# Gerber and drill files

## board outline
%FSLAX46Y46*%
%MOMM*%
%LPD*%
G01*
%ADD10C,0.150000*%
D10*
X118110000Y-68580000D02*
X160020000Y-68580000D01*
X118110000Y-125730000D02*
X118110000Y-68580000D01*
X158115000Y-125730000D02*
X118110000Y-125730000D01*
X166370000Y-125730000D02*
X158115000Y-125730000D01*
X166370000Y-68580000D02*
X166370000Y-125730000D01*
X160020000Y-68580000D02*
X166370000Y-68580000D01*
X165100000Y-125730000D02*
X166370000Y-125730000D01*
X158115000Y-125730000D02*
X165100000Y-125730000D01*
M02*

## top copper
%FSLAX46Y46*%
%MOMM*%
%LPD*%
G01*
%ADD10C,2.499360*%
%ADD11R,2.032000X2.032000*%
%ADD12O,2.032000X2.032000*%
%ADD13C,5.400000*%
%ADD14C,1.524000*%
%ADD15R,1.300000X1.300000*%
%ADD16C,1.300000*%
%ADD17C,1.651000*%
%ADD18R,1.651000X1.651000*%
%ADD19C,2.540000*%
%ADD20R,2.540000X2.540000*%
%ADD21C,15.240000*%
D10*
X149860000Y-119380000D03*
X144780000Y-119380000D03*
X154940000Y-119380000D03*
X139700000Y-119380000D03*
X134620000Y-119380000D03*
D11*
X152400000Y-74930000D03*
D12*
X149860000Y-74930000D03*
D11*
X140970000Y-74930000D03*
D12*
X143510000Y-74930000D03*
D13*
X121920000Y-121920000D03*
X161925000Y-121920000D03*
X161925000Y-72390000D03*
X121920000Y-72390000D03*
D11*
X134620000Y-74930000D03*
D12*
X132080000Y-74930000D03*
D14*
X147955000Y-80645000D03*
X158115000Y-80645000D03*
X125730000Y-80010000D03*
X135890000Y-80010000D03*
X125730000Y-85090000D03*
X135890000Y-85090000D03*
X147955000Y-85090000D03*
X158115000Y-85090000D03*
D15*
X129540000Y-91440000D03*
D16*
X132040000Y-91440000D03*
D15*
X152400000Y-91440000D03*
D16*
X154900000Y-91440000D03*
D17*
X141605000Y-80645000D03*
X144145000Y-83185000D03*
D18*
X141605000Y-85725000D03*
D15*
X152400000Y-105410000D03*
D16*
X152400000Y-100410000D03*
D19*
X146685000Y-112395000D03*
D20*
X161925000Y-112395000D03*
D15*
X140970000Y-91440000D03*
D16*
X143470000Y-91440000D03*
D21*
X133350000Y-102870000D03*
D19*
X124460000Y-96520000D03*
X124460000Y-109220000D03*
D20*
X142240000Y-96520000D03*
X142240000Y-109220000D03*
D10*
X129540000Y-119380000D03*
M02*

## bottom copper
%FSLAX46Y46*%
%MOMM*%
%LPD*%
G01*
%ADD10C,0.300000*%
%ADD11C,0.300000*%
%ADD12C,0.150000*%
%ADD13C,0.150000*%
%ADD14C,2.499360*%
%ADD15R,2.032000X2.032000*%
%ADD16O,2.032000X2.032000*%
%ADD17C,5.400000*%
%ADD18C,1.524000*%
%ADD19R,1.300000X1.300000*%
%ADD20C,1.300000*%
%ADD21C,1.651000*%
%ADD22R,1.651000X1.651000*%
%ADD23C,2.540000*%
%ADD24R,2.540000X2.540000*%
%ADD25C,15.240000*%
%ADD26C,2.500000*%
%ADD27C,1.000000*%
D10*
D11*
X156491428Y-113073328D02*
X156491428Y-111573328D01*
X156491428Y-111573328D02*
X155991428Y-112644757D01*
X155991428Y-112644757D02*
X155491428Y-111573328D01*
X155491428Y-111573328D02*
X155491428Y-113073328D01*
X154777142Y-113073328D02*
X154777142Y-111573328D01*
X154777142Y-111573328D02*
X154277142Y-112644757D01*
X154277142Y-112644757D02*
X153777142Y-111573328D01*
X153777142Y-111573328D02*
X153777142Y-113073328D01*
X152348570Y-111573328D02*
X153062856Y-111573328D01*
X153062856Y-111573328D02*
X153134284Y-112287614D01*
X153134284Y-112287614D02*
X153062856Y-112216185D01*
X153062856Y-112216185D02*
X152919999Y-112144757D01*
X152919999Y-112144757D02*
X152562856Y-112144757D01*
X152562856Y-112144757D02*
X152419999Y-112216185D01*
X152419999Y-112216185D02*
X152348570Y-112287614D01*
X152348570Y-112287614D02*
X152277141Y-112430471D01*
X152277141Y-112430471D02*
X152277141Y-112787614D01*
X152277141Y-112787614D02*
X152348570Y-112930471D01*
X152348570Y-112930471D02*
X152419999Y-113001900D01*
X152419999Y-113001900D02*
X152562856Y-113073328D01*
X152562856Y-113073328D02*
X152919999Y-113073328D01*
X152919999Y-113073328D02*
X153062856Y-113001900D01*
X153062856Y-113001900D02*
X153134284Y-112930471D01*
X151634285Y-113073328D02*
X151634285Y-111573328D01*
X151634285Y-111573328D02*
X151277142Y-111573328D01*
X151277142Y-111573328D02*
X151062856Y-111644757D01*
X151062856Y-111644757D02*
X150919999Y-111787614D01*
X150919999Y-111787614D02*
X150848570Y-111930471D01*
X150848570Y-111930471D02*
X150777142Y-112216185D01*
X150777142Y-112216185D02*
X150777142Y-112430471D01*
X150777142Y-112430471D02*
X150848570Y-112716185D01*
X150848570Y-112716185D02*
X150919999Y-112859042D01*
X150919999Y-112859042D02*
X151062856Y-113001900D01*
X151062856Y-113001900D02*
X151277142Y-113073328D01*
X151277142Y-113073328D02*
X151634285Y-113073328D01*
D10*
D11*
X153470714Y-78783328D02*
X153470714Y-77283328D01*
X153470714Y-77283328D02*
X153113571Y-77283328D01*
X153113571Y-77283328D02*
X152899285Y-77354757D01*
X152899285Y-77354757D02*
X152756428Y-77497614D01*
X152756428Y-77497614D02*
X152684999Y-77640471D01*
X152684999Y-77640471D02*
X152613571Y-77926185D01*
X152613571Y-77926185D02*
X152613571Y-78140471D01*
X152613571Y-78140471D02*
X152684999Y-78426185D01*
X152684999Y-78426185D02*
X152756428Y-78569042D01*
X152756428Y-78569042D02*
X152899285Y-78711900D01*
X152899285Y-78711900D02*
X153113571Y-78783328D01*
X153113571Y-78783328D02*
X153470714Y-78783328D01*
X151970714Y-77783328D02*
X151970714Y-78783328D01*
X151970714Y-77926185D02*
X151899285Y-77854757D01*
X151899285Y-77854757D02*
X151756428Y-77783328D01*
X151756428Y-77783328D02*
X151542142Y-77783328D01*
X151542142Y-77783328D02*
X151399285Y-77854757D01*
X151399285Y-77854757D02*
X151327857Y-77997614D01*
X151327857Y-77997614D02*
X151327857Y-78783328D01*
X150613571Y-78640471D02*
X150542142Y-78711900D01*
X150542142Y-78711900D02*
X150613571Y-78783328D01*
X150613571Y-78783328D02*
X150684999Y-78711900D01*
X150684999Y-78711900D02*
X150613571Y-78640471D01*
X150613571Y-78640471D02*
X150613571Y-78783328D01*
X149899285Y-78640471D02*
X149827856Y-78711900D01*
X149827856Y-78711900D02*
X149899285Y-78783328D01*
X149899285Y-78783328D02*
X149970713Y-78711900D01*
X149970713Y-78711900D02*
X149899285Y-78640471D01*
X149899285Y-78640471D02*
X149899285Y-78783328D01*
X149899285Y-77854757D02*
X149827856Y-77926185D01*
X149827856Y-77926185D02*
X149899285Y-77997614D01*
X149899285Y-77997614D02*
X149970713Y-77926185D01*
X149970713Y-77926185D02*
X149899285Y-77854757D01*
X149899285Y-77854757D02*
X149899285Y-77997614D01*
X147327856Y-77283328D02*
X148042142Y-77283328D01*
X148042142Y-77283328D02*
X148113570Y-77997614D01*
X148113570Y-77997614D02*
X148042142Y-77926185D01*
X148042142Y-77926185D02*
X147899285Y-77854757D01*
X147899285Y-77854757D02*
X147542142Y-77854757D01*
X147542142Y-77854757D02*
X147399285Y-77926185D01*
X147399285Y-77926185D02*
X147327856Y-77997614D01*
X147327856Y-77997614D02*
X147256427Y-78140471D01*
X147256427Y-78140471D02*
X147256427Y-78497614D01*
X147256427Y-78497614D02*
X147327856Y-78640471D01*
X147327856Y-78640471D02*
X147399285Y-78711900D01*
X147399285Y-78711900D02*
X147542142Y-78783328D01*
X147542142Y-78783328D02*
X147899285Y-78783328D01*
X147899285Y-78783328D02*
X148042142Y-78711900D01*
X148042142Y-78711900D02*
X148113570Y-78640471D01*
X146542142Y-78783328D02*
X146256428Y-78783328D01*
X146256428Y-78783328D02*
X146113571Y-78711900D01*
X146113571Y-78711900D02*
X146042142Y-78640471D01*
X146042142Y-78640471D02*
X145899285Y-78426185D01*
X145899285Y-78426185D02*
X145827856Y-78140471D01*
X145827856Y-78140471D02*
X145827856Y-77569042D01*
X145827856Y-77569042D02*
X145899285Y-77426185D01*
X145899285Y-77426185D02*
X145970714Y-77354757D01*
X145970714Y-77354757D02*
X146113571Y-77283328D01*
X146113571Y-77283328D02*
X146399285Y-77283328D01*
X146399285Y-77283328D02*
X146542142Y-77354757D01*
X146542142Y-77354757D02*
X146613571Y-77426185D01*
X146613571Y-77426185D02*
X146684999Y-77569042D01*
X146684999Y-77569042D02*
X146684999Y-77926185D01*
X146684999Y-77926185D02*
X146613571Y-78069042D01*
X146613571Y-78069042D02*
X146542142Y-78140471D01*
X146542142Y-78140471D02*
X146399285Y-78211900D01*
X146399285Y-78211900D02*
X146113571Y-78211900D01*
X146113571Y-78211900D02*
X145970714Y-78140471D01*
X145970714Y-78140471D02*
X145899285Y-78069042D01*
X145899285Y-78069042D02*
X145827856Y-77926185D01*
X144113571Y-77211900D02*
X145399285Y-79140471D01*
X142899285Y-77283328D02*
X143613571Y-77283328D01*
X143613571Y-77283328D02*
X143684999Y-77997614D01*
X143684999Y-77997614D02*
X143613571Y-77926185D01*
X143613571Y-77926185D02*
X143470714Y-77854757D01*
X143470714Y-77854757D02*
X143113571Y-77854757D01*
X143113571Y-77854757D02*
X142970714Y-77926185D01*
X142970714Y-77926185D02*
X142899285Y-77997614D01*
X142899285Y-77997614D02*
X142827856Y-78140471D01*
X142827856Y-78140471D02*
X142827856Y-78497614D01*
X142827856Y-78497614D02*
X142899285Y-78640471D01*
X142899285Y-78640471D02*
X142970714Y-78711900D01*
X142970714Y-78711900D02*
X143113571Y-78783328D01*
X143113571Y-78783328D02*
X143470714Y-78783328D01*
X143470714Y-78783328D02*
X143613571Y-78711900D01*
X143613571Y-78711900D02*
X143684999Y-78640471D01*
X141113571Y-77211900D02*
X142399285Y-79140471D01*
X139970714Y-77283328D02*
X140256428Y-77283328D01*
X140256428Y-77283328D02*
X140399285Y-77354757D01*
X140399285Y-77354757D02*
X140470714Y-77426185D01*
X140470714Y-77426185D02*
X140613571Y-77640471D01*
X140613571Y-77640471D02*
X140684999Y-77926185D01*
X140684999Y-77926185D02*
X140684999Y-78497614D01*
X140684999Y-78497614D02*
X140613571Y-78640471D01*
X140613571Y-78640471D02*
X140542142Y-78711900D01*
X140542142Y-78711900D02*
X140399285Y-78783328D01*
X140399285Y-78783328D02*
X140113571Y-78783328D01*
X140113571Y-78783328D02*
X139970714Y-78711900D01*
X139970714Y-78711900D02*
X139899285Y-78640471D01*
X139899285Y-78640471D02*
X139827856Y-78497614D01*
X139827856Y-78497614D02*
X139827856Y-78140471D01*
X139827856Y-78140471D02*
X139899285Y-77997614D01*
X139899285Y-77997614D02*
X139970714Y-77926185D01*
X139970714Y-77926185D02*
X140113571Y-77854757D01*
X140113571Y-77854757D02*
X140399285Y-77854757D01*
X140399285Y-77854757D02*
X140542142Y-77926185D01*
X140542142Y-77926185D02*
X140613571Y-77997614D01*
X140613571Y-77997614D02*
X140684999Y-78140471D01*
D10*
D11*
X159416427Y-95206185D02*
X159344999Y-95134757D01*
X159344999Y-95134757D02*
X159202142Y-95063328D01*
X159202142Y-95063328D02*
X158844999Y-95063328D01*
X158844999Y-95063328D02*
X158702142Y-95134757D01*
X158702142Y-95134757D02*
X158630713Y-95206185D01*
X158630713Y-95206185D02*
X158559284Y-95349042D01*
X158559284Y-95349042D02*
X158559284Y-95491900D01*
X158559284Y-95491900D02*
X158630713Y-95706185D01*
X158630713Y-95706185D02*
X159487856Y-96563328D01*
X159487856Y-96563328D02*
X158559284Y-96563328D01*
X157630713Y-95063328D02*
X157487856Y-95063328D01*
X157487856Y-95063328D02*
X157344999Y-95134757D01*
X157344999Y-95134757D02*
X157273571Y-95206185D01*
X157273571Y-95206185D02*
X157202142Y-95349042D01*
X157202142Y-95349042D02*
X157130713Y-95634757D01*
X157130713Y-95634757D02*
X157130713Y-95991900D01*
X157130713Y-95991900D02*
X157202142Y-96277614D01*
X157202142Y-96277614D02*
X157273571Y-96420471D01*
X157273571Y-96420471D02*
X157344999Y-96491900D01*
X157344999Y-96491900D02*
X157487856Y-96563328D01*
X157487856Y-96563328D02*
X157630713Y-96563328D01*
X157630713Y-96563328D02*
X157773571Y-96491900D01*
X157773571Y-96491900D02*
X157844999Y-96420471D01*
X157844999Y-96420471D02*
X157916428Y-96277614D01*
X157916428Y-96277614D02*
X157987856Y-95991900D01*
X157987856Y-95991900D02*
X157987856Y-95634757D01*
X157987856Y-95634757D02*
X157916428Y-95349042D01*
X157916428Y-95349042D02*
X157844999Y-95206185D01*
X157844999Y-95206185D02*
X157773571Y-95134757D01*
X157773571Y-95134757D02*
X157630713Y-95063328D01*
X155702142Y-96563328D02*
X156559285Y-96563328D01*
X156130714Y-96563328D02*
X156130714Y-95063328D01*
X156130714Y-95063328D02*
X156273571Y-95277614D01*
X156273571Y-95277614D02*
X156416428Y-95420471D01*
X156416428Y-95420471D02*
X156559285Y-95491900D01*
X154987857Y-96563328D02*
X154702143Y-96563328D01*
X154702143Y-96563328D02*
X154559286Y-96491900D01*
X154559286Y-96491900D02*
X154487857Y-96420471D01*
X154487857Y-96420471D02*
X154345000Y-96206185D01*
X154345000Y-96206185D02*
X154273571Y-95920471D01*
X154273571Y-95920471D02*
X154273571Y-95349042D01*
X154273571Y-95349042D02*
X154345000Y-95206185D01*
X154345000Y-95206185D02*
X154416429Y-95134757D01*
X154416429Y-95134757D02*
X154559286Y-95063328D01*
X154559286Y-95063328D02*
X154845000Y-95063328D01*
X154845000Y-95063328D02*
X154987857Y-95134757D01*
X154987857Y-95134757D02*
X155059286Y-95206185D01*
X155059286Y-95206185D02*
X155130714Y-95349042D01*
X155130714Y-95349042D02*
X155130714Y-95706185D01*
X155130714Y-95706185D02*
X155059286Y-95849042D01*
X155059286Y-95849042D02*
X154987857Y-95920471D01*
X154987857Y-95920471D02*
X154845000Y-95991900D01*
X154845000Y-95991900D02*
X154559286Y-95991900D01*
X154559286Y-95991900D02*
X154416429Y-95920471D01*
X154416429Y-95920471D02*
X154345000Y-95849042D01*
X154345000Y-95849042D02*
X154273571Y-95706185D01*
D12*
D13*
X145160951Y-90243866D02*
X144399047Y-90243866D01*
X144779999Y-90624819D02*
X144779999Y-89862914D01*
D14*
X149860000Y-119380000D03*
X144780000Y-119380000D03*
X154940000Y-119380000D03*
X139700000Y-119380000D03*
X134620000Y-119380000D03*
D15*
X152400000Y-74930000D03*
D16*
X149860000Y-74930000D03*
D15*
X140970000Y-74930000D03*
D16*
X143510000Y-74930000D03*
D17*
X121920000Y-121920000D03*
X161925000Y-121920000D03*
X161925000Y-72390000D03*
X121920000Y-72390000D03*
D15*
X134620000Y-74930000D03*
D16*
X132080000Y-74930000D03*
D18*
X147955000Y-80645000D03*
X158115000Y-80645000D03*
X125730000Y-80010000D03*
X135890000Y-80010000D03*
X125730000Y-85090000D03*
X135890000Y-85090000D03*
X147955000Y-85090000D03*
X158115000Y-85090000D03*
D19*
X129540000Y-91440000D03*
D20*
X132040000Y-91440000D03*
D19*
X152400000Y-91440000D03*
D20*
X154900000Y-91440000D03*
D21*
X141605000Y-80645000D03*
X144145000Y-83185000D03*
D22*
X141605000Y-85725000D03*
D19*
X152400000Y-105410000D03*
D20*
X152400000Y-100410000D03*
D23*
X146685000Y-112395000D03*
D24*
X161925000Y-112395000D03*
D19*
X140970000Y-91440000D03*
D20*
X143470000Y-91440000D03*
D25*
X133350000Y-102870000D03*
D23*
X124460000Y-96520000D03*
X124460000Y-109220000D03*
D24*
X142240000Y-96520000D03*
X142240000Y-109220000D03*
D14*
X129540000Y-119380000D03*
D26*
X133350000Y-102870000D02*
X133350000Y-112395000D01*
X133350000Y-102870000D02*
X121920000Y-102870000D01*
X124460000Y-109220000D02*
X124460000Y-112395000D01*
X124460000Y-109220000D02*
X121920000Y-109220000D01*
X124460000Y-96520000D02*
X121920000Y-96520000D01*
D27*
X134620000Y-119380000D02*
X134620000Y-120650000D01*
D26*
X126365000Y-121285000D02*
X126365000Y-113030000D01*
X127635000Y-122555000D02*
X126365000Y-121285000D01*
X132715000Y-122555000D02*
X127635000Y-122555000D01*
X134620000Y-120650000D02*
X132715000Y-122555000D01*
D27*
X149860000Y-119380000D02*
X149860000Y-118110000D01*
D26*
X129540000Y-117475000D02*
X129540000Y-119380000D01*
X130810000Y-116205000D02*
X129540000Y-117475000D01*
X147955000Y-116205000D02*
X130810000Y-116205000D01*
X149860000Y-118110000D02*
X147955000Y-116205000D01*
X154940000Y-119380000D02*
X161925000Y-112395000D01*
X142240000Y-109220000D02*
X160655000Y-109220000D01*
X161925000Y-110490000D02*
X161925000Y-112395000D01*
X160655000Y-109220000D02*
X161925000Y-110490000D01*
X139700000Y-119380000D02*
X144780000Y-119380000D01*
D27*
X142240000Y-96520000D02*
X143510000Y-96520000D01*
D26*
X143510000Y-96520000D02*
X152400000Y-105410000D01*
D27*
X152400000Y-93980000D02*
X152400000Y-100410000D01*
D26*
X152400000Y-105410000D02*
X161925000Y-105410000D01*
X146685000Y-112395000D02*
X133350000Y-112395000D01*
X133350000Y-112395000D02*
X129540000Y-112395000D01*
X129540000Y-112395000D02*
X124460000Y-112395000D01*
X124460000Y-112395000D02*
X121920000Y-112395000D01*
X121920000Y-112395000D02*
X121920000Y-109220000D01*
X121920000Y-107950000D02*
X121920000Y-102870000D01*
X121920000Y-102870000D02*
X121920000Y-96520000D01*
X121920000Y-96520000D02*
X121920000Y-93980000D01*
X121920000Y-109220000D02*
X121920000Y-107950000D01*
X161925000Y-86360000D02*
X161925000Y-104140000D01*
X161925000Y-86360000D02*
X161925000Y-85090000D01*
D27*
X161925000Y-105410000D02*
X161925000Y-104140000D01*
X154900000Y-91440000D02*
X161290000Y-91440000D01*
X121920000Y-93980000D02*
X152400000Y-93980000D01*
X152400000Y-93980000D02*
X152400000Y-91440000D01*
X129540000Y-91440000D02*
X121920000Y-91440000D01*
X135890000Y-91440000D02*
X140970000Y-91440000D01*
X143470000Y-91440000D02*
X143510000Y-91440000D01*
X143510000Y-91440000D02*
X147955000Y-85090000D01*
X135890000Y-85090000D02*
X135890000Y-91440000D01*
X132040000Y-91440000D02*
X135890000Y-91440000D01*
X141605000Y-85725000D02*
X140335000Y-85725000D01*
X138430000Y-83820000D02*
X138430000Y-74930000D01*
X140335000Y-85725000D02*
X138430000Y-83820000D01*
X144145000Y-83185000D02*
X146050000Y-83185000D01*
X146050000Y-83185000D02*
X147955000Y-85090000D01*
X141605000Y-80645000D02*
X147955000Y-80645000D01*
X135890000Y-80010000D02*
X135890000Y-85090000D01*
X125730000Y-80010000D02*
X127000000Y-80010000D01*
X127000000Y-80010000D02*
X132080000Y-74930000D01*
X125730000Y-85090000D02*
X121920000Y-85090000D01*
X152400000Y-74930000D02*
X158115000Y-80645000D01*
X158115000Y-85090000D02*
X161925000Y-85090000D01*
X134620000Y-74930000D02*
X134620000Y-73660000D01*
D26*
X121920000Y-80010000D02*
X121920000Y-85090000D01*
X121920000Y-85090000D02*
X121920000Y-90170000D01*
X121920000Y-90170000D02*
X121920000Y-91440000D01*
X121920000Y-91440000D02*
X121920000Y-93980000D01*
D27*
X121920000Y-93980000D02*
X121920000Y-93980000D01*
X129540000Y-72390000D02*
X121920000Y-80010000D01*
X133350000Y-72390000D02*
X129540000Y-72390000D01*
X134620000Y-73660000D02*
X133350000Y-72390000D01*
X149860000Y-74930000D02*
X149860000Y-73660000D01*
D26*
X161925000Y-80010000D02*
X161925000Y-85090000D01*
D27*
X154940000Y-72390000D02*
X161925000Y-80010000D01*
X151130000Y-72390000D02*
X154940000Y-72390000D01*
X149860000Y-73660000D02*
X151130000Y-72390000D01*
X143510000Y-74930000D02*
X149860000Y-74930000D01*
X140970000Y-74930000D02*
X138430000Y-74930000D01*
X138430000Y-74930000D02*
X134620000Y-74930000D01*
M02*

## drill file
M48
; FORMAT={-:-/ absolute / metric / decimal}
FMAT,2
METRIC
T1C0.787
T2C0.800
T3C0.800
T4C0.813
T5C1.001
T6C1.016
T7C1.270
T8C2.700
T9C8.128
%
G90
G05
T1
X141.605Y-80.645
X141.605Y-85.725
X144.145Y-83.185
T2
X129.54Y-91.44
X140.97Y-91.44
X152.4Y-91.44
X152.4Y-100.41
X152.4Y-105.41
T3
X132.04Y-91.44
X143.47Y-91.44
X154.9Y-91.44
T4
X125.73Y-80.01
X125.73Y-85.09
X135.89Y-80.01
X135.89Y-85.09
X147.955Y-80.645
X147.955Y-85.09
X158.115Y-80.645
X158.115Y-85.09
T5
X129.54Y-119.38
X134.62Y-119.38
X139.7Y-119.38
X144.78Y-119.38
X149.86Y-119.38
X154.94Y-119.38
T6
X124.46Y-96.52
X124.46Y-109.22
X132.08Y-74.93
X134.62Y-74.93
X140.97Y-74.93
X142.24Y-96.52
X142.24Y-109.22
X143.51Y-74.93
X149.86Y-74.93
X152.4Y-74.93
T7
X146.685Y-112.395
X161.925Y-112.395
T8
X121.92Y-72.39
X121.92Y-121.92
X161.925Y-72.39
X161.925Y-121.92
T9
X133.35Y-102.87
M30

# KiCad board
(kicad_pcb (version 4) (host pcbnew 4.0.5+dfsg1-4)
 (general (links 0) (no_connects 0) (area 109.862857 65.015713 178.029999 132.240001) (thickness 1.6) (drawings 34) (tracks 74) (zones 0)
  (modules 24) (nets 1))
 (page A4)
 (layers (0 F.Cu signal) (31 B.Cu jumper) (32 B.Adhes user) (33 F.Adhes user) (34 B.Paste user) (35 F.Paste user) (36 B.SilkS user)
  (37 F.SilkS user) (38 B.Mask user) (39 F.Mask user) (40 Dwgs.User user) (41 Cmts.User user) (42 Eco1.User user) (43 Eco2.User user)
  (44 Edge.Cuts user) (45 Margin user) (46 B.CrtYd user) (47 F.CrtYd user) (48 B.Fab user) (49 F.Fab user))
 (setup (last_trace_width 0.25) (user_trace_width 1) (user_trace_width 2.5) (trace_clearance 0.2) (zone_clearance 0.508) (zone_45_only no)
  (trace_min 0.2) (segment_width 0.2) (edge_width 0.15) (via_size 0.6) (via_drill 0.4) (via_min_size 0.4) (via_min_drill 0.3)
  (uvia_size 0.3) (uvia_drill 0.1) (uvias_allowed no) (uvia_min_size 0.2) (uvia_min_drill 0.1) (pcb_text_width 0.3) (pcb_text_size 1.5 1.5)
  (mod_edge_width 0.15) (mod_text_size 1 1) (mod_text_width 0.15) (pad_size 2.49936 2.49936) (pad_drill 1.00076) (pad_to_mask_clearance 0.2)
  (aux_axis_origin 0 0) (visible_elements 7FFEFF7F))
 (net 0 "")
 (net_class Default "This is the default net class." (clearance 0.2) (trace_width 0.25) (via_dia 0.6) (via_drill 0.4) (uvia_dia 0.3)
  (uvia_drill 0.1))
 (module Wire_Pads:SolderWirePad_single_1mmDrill (layer F.Cu) (at 149.86 119.38)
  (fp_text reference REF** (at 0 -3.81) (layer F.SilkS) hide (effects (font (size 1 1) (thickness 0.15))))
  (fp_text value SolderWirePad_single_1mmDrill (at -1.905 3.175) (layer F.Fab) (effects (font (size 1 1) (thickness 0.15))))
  (pad 2 thru_hole circle (at 0 0) (size 2.49936 2.49936) (drill 1.00076) (layers *.Cu *.Mask)))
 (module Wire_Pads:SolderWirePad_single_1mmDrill (layer F.Cu) (at 144.78 119.38)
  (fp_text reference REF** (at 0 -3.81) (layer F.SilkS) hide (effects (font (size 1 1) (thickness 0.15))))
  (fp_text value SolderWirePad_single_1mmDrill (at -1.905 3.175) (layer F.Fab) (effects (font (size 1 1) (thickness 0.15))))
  (pad 1 thru_hole circle (at 0 0) (size 2.49936 2.49936) (drill 1.00076) (layers *.Cu *.Mask)))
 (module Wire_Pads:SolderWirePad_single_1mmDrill (layer F.Cu) (at 154.94 119.38)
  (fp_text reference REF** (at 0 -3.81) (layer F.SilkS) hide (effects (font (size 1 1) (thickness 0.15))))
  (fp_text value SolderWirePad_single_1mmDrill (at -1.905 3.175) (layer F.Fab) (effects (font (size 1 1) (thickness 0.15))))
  (pad 3 thru_hole circle (at 0 0) (size 2.49936 2.49936) (drill 1.00076) (layers *.Cu *.Mask)))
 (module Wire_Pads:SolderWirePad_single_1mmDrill (layer F.Cu) (at 139.7 119.38)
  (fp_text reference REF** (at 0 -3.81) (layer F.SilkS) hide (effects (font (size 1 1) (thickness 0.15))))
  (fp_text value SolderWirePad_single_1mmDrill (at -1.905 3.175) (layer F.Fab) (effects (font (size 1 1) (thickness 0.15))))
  (pad 3 thru_hole circle (at 0 0) (size 2.49936 2.49936) (drill 1.00076) (layers *.Cu *.Mask)))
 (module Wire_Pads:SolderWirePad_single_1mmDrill (layer F.Cu) (at 134.62 119.38)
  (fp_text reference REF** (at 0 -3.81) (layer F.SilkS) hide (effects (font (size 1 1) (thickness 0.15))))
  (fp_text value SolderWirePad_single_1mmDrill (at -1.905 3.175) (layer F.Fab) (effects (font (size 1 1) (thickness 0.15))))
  (pad 2 thru_hole circle (at 0 0) (size 2.49936 2.49936) (drill 1.00076) (layers *.Cu *.Mask)))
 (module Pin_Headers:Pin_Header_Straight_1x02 (layer F.Cu) (at 152.4 74.93 270)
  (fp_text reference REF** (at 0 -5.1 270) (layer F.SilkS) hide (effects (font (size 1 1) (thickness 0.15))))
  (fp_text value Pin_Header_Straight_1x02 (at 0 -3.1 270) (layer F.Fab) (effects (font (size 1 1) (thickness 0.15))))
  (pad 1 thru_hole rect (at 0 0 270) (size 2.032 2.032) (drill 1.016) (layers *.Cu *.Mask))
  (pad 2 thru_hole oval (at 0 2.54 270) (size 2.032 2.032) (drill 1.016) (layers *.Cu *.Mask)))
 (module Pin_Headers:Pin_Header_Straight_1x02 (layer F.Cu) (at 140.97 74.93 90)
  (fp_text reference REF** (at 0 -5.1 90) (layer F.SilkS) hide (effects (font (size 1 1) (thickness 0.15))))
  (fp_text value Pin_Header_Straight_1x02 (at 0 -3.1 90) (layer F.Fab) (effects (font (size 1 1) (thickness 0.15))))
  (pad 1 thru_hole rect (at 0 0 90) (size 2.032 2.032) (drill 1.016) (layers *.Cu *.Mask))
  (pad 2 thru_hole oval (at 0 2.54 90) (size 2.032 2.032) (drill 1.016) (layers *.Cu *.Mask)))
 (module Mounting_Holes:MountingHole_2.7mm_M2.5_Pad (layer F.Cu) (at 121.92 121.92)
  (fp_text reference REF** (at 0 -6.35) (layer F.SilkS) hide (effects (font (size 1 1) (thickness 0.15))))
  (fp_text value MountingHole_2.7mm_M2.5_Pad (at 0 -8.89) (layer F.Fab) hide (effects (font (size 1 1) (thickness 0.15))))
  (pad 1 thru_hole circle (at 0 0) (size 5.4 5.4) (drill 2.7) (layers *.Cu *.Mask)))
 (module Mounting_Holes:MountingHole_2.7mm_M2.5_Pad (layer F.Cu) (at 161.925 121.92)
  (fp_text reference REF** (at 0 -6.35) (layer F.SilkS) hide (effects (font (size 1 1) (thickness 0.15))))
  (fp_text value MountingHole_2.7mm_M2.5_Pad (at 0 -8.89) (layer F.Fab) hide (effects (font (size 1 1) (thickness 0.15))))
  (pad 1 thru_hole circle (at 0 0) (size 5.4 5.4) (drill 2.7) (layers *.Cu *.Mask)))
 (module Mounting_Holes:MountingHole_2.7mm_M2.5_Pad (layer F.Cu) (at 161.925 72.39)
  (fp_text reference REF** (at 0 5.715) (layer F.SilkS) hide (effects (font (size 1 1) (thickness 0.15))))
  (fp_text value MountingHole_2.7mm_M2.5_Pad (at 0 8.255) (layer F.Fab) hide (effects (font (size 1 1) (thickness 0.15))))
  (pad 1 thru_hole circle (at 0 0) (size 5.4 5.4) (drill 2.7) (layers *.Cu *.Mask)))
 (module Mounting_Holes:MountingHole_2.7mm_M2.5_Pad (layer F.Cu) (at 121.92 72.39)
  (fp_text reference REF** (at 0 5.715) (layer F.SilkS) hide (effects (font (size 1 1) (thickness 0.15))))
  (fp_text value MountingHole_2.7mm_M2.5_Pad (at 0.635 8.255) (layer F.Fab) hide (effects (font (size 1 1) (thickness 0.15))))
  (pad 1 thru_hole circle (at 0 0) (size 5.4 5.4) (drill 2.7) (layers *.Cu *.Mask)))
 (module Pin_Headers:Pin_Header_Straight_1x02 (layer F.Cu) (at 134.62 74.93 270)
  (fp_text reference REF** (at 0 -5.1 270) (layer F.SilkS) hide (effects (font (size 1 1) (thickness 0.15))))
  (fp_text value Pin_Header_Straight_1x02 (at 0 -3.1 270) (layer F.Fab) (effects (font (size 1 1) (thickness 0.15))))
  (pad 1 thru_hole rect (at 0 0 270) (size 2.032 2.032) (drill 1.016) (layers *.Cu *.Mask))
  (pad 2 thru_hole oval (at 0 2.54 270) (size 2.032 2.032) (drill 1.016) (layers *.Cu *.Mask)))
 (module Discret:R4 (layer F.Cu) (at 153.035 80.645)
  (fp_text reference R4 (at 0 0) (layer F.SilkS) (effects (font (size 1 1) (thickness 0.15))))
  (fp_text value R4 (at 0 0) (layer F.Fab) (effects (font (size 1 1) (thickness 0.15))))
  (pad 1 thru_hole circle (at -5.08 0) (size 1.524 1.524) (drill 0.8128) (layers *.Cu *.Mask))
  (pad 2 thru_hole circle (at 5.08 0) (size 1.524 1.524) (drill 0.8128) (layers *.Cu *.Mask)))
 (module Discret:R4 (layer F.Cu) (at 130.81 80.01)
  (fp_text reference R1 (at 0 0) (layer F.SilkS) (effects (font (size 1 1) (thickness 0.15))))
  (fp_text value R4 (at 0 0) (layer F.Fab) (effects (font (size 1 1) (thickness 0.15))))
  (pad 1 thru_hole circle (at -5.08 0) (size 1.524 1.524) (drill 0.8128) (layers *.Cu *.Mask))
  (pad 2 thru_hole circle (at 5.08 0) (size 1.524 1.524) (drill 0.8128) (layers *.Cu *.Mask)))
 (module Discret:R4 (layer F.Cu) (at 130.81 85.09)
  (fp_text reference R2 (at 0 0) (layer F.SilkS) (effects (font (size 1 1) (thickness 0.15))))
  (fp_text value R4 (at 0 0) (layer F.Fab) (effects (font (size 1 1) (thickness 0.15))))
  (pad 1 thru_hole circle (at -5.08 0) (size 1.524 1.524) (drill 0.8128) (layers *.Cu *.Mask))
  (pad 2 thru_hole circle (at 5.08 0) (size 1.524 1.524) (drill 0.8128) (layers *.Cu *.Mask)))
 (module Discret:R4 (layer F.Cu) (at 153.035 85.09)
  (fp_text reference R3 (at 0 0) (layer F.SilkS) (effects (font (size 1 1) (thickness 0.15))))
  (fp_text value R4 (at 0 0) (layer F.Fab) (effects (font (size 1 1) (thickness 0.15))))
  (pad 1 thru_hole circle (at -5.08 0) (size 1.524 1.524) (drill 0.8128) (layers *.Cu *.Mask))
  (pad 2 thru_hole circle (at 5.08 0) (size 1.524 1.524) (drill 0.8128) (layers *.Cu *.Mask)))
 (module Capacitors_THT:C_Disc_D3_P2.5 (layer F.Cu) (at 129.54 91.44)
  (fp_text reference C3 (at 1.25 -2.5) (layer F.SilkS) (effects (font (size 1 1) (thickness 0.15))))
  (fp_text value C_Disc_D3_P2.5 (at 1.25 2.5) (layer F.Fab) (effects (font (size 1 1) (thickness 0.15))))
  (pad 1 thru_hole rect (at 0 0) (size 1.3 1.3) (drill 0.8) (layers *.Cu *.Mask))
  (pad 2 thru_hole circle (at 2.5 0) (size 1.3 1.3) (drill 0.8001) (layers *.Cu *.Mask)))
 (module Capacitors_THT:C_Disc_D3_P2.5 (layer F.Cu) (at 152.4 91.44)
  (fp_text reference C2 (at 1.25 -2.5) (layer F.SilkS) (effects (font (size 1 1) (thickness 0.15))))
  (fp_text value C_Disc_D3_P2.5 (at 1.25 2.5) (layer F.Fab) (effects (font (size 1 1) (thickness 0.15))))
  (pad 1 thru_hole rect (at 0 0) (size 1.3 1.3) (drill 0.8) (layers *.Cu *.Mask))
  (pad 2 thru_hole circle (at 2.5 0) (size 1.3 1.3) (drill 0.8001) (layers *.Cu *.Mask)))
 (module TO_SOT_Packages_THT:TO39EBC (layer F.Cu) (at 141.605 85.725 90)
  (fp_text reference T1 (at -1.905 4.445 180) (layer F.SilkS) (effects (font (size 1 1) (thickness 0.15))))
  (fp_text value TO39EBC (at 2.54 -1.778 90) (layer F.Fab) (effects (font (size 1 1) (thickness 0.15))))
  (pad 3 thru_hole circle (at 5.08 0 90) (size 1.651 1.651) (drill 0.7874) (layers *.Cu *.Mask))
  (pad 2 thru_hole circle (at 2.54 2.54 90) (size 1.651 1.651) (drill 0.7874) (layers *.Cu *.Mask))
  (pad 1 thru_hole rect (at 0 0 90) (size 1.651 1.651) (drill 0.7874) (layers *.Cu *.Mask)))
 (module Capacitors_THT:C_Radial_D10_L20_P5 (layer F.Cu) (at 152.4 105.41 90)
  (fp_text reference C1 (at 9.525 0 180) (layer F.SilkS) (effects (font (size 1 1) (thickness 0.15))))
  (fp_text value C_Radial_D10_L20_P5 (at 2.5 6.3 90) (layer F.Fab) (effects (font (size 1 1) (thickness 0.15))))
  (pad 1 thru_hole rect (at 0 0 90) (size 1.3 1.3) (drill 0.8) (layers *.Cu *.Mask))
  (pad 2 thru_hole circle (at 5 0 90) (size 1.3 1.3) (drill 0.8) (layers *.Cu *.Mask)))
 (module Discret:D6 (layer F.Cu) (at 154.305 112.395)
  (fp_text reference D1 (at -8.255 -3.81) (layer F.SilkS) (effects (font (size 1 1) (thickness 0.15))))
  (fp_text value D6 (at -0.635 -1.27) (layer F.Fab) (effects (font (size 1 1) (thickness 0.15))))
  (pad 2 thru_hole circle (at -7.62 0) (size 2.54 2.54) (drill 1.27) (layers *.Cu *.Mask))
  (pad 1 thru_hole rect (at 7.62 0) (size 2.54 2.54) (drill 1.27) (layers *.Cu *.Mask)))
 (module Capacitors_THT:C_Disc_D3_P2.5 (layer F.Cu) (at 140.97 91.44)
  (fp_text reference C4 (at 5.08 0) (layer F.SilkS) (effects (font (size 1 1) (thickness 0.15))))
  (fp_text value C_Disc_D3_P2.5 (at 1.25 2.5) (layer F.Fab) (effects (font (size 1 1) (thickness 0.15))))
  (pad 1 thru_hole rect (at 0 0) (size 1.3 1.3) (drill 0.8) (layers *.Cu *.Mask))
  (pad 2 thru_hole circle (at 2.5 0) (size 1.3 1.3) (drill 0.8001) (layers *.Cu *.Mask)))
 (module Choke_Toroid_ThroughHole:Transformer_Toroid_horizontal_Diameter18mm (layer F.Cu) (at 133.35 102.87)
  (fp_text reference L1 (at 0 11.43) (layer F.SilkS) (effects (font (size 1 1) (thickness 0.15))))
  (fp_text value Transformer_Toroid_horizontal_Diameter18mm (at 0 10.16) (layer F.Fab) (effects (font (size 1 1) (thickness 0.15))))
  (pad "" thru_hole circle (at 0 0) (size 15.24 15.24) (drill 8.128) (layers *.Cu *.SilkS *.Mask))
  (pad 1 thru_hole circle (at -8.89 -6.35) (size 2.54 2.54) (drill 1.016) (layers *.Cu *.SilkS *.Mask))
  (pad 2 thru_hole circle (at -8.89 6.35) (size 2.54 2.54) (drill 1.016) (layers *.Cu *.SilkS *.Mask))
  (pad 3 thru_hole rect (at 8.89 -6.35) (size 2.54 2.54) (drill 1.016) (layers *.Cu *.SilkS *.Mask))
  (pad 4 thru_hole rect (at 8.89 6.35) (size 2.54 2.54) (drill 1.016) (layers *.Cu *.SilkS *.Mask)))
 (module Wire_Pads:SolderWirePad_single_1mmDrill (layer F.Cu) (at 129.54 119.38)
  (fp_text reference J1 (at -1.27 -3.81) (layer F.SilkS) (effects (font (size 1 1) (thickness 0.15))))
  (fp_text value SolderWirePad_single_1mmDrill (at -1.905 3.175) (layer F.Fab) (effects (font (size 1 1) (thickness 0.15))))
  (pad 1 thru_hole circle (at 0 0) (size 2.49936 2.49936) (drill 1.00076) (layers *.Cu *.Mask)))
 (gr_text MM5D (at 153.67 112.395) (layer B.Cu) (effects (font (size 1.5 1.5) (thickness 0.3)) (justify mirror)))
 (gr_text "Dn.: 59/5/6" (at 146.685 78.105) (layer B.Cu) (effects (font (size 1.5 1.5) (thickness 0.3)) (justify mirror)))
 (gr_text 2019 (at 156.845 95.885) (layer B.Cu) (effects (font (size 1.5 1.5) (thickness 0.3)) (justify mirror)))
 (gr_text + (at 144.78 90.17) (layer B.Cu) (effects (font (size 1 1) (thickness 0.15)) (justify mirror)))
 (gr_line (start 118.11 68.58) (end 160.02 68.58) (angle 90) (layer Edge.Cuts) (width 0.15))
 (gr_line (start 118.11 125.73) (end 118.11 68.58) (angle 90) (layer Edge.Cuts) (width 0.15))
 (gr_line (start 158.115 125.73) (end 118.11 125.73) (angle 90) (layer Edge.Cuts) (width 0.15))
 (gr_line (start 166.37 125.73) (end 158.115 125.73) (angle 90) (layer Edge.Cuts) (width 0.15))
 (gr_line (start 166.37 68.58) (end 166.37 125.73) (angle 90) (layer Edge.Cuts) (width 0.15))
 (gr_line (start 160.02 68.58) (end 166.37 68.58) (angle 90) (layer Edge.Cuts) (width 0.15))
 (gr_line (start 165.1 125.73) (end 166.37 125.73) (angle 90) (layer Edge.Cuts) (width 0.15))
 (gr_line (start 158.115 125.73) (end 165.1 125.73) (angle 90) (layer Edge.Cuts) (width 0.15))
 (segment (start 133.35 102.87) (end 133.35 112.395) (width 2.5) (layer B.Cu) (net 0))
 (segment (start 133.35 102.87) (end 121.92 102.87) (width 2.5) (layer B.Cu) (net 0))
 (segment (start 124.46 109.22) (end 124.46 112.395) (width 2.5) (layer B.Cu) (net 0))
 (segment (start 124.46 109.22) (end 121.92 109.22) (width 2.5) (layer B.Cu) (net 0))
 (segment (start 124.46 96.52) (end 121.92 96.52) (width 2.5) (layer B.Cu) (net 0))
 (segment (start 134.62 119.38) (end 134.62 120.65) (width 1) (layer B.Cu) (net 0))
 (segment (start 126.365 121.285) (end 126.365 113.03) (width 2.5) (layer B.Cu) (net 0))
 (segment (start 127.635 122.555) (end 126.365 121.285) (width 2.5) (layer B.Cu) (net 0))
 (segment (start 132.715 122.555) (end 127.635 122.555) (width 2.5) (layer B.Cu) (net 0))
 (segment (start 134.62 120.65) (end 132.715 122.555) (width 2.5) (layer B.Cu) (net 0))
 (segment (start 149.86 119.38) (end 149.86 118.11) (width 1) (layer B.Cu) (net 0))
 (segment (start 129.54 117.475) (end 129.54 119.38) (width 2.5) (layer B.Cu) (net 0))
 (segment (start 130.81 116.205) (end 129.54 117.475) (width 2.5) (layer B.Cu) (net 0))
 (segment (start 147.955 116.205) (end 130.81 116.205) (width 2.5) (layer B.Cu) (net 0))
 (segment (start 149.86 118.11) (end 147.955 116.205) (width 2.5) (layer B.Cu) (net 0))
 (segment (start 154.94 119.38) (end 161.925 112.395) (width 2.5) (layer B.Cu) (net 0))
 (segment (start 142.24 109.22) (end 160.655 109.22) (width 2.5) (layer B.Cu) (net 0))
 (segment (start 161.925 110.49) (end 161.925 112.395) (width 2.5) (layer B.Cu) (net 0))
 (segment (start 160.655 109.22) (end 161.925 110.49) (width 2.5) (layer B.Cu) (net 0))
 (segment (start 139.7 119.38) (end 144.78 119.38) (width 2.5) (layer B.Cu) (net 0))
 (segment (start 142.24 96.52) (end 143.51 96.52) (width 1) (layer B.Cu) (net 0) (status 30))
 (segment (start 143.51 96.52) (end 152.4 105.41) (width 2.5) (layer B.Cu) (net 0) (status 20))
 (segment (start 152.4 93.98) (end 152.4 100.41) (width 1) (layer B.Cu) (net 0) (status 20))
 (segment (start 152.4 105.41) (end 161.925 105.41) (width 2.5) (layer B.Cu) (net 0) (status 10))
 (segment (start 146.685 112.395) (end 133.35 112.395) (width 2.5) (layer B.Cu) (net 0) (status 10))
 (segment (start 133.35 112.395) (end 129.54 112.395) (width 2.5) (layer B.Cu) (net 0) (status 10))
 (segment (start 129.54 112.395) (end 124.46 112.395) (width 2.5) (layer B.Cu) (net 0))
 (segment (start 124.46 112.395) (end 121.92 112.395) (width 2.5) (layer B.Cu) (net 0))
 (segment (start 121.92 112.395) (end 121.92 109.22) (width 2.5) (layer B.Cu) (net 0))
 (segment (start 121.92 107.95) (end 121.92 102.87) (width 2.5) (layer B.Cu) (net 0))
 (segment (start 121.92 102.87) (end 121.92 96.52) (width 2.5) (layer B.Cu) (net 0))
 (segment (start 121.92 96.52) (end 121.92 93.98) (width 2.5) (layer B.Cu) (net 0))
 (segment (start 121.92 109.22) (end 121.92 107.95) (width 2.5) (layer B.Cu) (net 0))
 (segment (start 161.925 86.36) (end 161.925 104.14) (width 2.5) (layer B.Cu) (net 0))
 (segment (start 161.925 86.36) (end 161.925 85.09) (width 2.5) (layer B.Cu) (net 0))
 (segment (start 161.925 105.41) (end 161.925 104.14) (width 1) (layer B.Cu) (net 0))
 (segment (start 154.9 91.44) (end 161.29 91.44) (width 1) (layer B.Cu) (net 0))
 (segment (start 121.92 93.98) (end 152.4 93.98) (width 1) (layer B.Cu) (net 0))
 (segment (start 152.4 93.98) (end 152.4 91.44) (width 1) (layer B.Cu) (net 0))
 (segment (start 129.54 91.44) (end 121.92 91.44) (width 1) (layer B.Cu) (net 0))
 (segment (start 135.89 91.44) (end 140.97 91.44) (width 1) (layer B.Cu) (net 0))
 (segment (start 143.47 91.44) (end 143.51 91.44) (width 1) (layer B.Cu) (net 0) (status 30))
 (segment (start 143.51 91.44) (end 147.955 85.09) (width 1) (layer B.Cu) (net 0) (status 10))
 (segment (start 135.89 85.09) (end 135.89 91.44) (width 1) (layer B.Cu) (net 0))
 (segment (start 132.04 91.44) (end 135.89 91.44) (width 1) (layer B.Cu) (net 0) (status 10))
 (segment (start 141.605 85.725) (end 140.335 85.725) (width 1) (layer B.Cu) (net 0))
 (segment (start 138.43 83.82) (end 138.43 74.93) (width 1) (layer B.Cu) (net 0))
 (segment (start 140.335 85.725) (end 138.43 83.82) (width 1) (layer B.Cu) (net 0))
 (segment (start 144.145 83.185) (end 146.05 83.185) (width 1) (layer B.Cu) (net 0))
 (segment (start 146.05 83.185) (end 147.955 85.09) (width 1) (layer B.Cu) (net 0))
 (segment (start 141.605 80.645) (end 147.955 80.645) (width 1) (layer B.Cu) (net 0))
 (segment (start 135.89 80.01) (end 135.89 85.09) (width 1) (layer B.Cu) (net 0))
 (segment (start 125.73 80.01) (end 127 80.01) (width 1) (layer B.Cu) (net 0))
 (segment (start 127 80.01) (end 132.08 74.93) (width 1) (layer B.Cu) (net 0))
 (segment (start 125.73 85.09) (end 121.92 85.09) (width 1) (layer B.Cu) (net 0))
 (segment (start 152.4 74.93) (end 158.115 80.645) (width 1) (layer B.Cu) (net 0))
 (segment (start 158.115 85.09) (end 161.925 85.09) (width 1) (layer B.Cu) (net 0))
 (segment (start 134.62 74.93) (end 134.62 73.66) (width 1) (layer B.Cu) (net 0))
 (segment (start 121.92 80.01) (end 121.92 85.09) (width 2.5) (layer B.Cu) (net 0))
 (segment (start 121.92 85.09) (end 121.92 90.17) (width 2.5) (layer B.Cu) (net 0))
 (segment (start 121.92 90.17) (end 121.92 91.44) (width 2.5) (layer B.Cu) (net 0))
 (segment (start 121.92 91.44) (end 121.92 93.98) (width 2.5) (layer B.Cu) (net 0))
 (segment (start 121.92 93.98) (end 121.92 93.98) (width 1) (layer B.Cu) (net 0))
 (segment (start 129.54 72.39) (end 121.92 80.01) (width 1) (layer B.Cu) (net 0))
 (segment (start 133.35 72.39) (end 129.54 72.39) (width 1) (layer B.Cu) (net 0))
 (segment (start 134.62 73.66) (end 133.35 72.39) (width 1) (layer B.Cu) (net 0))
 (segment (start 149.86 74.93) (end 149.86 73.66) (width 1) (layer B.Cu) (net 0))
 (segment (start 161.925 80.01) (end 161.925 85.09) (width 2.5) (layer B.Cu) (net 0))
 (segment (start 154.94 72.39) (end 161.925 80.01) (width 1) (layer B.Cu) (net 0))
 (segment (start 151.13 72.39) (end 154.94 72.39) (width 1) (layer B.Cu) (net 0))
 (segment (start 149.86 73.66) (end 151.13 72.39) (width 1) (layer B.Cu) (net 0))
 (segment (start 143.51 74.93) (end 149.86 74.93) (width 1) (layer B.Cu) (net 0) (status 20))
 (segment (start 140.97 74.93) (end 138.43 74.93) (width 1) (layer B.Cu) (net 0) (status 20))
 (segment (start 138.43 74.93) (end 134.62 74.93) (width 1) (layer B.Cu) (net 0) (status 20)))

